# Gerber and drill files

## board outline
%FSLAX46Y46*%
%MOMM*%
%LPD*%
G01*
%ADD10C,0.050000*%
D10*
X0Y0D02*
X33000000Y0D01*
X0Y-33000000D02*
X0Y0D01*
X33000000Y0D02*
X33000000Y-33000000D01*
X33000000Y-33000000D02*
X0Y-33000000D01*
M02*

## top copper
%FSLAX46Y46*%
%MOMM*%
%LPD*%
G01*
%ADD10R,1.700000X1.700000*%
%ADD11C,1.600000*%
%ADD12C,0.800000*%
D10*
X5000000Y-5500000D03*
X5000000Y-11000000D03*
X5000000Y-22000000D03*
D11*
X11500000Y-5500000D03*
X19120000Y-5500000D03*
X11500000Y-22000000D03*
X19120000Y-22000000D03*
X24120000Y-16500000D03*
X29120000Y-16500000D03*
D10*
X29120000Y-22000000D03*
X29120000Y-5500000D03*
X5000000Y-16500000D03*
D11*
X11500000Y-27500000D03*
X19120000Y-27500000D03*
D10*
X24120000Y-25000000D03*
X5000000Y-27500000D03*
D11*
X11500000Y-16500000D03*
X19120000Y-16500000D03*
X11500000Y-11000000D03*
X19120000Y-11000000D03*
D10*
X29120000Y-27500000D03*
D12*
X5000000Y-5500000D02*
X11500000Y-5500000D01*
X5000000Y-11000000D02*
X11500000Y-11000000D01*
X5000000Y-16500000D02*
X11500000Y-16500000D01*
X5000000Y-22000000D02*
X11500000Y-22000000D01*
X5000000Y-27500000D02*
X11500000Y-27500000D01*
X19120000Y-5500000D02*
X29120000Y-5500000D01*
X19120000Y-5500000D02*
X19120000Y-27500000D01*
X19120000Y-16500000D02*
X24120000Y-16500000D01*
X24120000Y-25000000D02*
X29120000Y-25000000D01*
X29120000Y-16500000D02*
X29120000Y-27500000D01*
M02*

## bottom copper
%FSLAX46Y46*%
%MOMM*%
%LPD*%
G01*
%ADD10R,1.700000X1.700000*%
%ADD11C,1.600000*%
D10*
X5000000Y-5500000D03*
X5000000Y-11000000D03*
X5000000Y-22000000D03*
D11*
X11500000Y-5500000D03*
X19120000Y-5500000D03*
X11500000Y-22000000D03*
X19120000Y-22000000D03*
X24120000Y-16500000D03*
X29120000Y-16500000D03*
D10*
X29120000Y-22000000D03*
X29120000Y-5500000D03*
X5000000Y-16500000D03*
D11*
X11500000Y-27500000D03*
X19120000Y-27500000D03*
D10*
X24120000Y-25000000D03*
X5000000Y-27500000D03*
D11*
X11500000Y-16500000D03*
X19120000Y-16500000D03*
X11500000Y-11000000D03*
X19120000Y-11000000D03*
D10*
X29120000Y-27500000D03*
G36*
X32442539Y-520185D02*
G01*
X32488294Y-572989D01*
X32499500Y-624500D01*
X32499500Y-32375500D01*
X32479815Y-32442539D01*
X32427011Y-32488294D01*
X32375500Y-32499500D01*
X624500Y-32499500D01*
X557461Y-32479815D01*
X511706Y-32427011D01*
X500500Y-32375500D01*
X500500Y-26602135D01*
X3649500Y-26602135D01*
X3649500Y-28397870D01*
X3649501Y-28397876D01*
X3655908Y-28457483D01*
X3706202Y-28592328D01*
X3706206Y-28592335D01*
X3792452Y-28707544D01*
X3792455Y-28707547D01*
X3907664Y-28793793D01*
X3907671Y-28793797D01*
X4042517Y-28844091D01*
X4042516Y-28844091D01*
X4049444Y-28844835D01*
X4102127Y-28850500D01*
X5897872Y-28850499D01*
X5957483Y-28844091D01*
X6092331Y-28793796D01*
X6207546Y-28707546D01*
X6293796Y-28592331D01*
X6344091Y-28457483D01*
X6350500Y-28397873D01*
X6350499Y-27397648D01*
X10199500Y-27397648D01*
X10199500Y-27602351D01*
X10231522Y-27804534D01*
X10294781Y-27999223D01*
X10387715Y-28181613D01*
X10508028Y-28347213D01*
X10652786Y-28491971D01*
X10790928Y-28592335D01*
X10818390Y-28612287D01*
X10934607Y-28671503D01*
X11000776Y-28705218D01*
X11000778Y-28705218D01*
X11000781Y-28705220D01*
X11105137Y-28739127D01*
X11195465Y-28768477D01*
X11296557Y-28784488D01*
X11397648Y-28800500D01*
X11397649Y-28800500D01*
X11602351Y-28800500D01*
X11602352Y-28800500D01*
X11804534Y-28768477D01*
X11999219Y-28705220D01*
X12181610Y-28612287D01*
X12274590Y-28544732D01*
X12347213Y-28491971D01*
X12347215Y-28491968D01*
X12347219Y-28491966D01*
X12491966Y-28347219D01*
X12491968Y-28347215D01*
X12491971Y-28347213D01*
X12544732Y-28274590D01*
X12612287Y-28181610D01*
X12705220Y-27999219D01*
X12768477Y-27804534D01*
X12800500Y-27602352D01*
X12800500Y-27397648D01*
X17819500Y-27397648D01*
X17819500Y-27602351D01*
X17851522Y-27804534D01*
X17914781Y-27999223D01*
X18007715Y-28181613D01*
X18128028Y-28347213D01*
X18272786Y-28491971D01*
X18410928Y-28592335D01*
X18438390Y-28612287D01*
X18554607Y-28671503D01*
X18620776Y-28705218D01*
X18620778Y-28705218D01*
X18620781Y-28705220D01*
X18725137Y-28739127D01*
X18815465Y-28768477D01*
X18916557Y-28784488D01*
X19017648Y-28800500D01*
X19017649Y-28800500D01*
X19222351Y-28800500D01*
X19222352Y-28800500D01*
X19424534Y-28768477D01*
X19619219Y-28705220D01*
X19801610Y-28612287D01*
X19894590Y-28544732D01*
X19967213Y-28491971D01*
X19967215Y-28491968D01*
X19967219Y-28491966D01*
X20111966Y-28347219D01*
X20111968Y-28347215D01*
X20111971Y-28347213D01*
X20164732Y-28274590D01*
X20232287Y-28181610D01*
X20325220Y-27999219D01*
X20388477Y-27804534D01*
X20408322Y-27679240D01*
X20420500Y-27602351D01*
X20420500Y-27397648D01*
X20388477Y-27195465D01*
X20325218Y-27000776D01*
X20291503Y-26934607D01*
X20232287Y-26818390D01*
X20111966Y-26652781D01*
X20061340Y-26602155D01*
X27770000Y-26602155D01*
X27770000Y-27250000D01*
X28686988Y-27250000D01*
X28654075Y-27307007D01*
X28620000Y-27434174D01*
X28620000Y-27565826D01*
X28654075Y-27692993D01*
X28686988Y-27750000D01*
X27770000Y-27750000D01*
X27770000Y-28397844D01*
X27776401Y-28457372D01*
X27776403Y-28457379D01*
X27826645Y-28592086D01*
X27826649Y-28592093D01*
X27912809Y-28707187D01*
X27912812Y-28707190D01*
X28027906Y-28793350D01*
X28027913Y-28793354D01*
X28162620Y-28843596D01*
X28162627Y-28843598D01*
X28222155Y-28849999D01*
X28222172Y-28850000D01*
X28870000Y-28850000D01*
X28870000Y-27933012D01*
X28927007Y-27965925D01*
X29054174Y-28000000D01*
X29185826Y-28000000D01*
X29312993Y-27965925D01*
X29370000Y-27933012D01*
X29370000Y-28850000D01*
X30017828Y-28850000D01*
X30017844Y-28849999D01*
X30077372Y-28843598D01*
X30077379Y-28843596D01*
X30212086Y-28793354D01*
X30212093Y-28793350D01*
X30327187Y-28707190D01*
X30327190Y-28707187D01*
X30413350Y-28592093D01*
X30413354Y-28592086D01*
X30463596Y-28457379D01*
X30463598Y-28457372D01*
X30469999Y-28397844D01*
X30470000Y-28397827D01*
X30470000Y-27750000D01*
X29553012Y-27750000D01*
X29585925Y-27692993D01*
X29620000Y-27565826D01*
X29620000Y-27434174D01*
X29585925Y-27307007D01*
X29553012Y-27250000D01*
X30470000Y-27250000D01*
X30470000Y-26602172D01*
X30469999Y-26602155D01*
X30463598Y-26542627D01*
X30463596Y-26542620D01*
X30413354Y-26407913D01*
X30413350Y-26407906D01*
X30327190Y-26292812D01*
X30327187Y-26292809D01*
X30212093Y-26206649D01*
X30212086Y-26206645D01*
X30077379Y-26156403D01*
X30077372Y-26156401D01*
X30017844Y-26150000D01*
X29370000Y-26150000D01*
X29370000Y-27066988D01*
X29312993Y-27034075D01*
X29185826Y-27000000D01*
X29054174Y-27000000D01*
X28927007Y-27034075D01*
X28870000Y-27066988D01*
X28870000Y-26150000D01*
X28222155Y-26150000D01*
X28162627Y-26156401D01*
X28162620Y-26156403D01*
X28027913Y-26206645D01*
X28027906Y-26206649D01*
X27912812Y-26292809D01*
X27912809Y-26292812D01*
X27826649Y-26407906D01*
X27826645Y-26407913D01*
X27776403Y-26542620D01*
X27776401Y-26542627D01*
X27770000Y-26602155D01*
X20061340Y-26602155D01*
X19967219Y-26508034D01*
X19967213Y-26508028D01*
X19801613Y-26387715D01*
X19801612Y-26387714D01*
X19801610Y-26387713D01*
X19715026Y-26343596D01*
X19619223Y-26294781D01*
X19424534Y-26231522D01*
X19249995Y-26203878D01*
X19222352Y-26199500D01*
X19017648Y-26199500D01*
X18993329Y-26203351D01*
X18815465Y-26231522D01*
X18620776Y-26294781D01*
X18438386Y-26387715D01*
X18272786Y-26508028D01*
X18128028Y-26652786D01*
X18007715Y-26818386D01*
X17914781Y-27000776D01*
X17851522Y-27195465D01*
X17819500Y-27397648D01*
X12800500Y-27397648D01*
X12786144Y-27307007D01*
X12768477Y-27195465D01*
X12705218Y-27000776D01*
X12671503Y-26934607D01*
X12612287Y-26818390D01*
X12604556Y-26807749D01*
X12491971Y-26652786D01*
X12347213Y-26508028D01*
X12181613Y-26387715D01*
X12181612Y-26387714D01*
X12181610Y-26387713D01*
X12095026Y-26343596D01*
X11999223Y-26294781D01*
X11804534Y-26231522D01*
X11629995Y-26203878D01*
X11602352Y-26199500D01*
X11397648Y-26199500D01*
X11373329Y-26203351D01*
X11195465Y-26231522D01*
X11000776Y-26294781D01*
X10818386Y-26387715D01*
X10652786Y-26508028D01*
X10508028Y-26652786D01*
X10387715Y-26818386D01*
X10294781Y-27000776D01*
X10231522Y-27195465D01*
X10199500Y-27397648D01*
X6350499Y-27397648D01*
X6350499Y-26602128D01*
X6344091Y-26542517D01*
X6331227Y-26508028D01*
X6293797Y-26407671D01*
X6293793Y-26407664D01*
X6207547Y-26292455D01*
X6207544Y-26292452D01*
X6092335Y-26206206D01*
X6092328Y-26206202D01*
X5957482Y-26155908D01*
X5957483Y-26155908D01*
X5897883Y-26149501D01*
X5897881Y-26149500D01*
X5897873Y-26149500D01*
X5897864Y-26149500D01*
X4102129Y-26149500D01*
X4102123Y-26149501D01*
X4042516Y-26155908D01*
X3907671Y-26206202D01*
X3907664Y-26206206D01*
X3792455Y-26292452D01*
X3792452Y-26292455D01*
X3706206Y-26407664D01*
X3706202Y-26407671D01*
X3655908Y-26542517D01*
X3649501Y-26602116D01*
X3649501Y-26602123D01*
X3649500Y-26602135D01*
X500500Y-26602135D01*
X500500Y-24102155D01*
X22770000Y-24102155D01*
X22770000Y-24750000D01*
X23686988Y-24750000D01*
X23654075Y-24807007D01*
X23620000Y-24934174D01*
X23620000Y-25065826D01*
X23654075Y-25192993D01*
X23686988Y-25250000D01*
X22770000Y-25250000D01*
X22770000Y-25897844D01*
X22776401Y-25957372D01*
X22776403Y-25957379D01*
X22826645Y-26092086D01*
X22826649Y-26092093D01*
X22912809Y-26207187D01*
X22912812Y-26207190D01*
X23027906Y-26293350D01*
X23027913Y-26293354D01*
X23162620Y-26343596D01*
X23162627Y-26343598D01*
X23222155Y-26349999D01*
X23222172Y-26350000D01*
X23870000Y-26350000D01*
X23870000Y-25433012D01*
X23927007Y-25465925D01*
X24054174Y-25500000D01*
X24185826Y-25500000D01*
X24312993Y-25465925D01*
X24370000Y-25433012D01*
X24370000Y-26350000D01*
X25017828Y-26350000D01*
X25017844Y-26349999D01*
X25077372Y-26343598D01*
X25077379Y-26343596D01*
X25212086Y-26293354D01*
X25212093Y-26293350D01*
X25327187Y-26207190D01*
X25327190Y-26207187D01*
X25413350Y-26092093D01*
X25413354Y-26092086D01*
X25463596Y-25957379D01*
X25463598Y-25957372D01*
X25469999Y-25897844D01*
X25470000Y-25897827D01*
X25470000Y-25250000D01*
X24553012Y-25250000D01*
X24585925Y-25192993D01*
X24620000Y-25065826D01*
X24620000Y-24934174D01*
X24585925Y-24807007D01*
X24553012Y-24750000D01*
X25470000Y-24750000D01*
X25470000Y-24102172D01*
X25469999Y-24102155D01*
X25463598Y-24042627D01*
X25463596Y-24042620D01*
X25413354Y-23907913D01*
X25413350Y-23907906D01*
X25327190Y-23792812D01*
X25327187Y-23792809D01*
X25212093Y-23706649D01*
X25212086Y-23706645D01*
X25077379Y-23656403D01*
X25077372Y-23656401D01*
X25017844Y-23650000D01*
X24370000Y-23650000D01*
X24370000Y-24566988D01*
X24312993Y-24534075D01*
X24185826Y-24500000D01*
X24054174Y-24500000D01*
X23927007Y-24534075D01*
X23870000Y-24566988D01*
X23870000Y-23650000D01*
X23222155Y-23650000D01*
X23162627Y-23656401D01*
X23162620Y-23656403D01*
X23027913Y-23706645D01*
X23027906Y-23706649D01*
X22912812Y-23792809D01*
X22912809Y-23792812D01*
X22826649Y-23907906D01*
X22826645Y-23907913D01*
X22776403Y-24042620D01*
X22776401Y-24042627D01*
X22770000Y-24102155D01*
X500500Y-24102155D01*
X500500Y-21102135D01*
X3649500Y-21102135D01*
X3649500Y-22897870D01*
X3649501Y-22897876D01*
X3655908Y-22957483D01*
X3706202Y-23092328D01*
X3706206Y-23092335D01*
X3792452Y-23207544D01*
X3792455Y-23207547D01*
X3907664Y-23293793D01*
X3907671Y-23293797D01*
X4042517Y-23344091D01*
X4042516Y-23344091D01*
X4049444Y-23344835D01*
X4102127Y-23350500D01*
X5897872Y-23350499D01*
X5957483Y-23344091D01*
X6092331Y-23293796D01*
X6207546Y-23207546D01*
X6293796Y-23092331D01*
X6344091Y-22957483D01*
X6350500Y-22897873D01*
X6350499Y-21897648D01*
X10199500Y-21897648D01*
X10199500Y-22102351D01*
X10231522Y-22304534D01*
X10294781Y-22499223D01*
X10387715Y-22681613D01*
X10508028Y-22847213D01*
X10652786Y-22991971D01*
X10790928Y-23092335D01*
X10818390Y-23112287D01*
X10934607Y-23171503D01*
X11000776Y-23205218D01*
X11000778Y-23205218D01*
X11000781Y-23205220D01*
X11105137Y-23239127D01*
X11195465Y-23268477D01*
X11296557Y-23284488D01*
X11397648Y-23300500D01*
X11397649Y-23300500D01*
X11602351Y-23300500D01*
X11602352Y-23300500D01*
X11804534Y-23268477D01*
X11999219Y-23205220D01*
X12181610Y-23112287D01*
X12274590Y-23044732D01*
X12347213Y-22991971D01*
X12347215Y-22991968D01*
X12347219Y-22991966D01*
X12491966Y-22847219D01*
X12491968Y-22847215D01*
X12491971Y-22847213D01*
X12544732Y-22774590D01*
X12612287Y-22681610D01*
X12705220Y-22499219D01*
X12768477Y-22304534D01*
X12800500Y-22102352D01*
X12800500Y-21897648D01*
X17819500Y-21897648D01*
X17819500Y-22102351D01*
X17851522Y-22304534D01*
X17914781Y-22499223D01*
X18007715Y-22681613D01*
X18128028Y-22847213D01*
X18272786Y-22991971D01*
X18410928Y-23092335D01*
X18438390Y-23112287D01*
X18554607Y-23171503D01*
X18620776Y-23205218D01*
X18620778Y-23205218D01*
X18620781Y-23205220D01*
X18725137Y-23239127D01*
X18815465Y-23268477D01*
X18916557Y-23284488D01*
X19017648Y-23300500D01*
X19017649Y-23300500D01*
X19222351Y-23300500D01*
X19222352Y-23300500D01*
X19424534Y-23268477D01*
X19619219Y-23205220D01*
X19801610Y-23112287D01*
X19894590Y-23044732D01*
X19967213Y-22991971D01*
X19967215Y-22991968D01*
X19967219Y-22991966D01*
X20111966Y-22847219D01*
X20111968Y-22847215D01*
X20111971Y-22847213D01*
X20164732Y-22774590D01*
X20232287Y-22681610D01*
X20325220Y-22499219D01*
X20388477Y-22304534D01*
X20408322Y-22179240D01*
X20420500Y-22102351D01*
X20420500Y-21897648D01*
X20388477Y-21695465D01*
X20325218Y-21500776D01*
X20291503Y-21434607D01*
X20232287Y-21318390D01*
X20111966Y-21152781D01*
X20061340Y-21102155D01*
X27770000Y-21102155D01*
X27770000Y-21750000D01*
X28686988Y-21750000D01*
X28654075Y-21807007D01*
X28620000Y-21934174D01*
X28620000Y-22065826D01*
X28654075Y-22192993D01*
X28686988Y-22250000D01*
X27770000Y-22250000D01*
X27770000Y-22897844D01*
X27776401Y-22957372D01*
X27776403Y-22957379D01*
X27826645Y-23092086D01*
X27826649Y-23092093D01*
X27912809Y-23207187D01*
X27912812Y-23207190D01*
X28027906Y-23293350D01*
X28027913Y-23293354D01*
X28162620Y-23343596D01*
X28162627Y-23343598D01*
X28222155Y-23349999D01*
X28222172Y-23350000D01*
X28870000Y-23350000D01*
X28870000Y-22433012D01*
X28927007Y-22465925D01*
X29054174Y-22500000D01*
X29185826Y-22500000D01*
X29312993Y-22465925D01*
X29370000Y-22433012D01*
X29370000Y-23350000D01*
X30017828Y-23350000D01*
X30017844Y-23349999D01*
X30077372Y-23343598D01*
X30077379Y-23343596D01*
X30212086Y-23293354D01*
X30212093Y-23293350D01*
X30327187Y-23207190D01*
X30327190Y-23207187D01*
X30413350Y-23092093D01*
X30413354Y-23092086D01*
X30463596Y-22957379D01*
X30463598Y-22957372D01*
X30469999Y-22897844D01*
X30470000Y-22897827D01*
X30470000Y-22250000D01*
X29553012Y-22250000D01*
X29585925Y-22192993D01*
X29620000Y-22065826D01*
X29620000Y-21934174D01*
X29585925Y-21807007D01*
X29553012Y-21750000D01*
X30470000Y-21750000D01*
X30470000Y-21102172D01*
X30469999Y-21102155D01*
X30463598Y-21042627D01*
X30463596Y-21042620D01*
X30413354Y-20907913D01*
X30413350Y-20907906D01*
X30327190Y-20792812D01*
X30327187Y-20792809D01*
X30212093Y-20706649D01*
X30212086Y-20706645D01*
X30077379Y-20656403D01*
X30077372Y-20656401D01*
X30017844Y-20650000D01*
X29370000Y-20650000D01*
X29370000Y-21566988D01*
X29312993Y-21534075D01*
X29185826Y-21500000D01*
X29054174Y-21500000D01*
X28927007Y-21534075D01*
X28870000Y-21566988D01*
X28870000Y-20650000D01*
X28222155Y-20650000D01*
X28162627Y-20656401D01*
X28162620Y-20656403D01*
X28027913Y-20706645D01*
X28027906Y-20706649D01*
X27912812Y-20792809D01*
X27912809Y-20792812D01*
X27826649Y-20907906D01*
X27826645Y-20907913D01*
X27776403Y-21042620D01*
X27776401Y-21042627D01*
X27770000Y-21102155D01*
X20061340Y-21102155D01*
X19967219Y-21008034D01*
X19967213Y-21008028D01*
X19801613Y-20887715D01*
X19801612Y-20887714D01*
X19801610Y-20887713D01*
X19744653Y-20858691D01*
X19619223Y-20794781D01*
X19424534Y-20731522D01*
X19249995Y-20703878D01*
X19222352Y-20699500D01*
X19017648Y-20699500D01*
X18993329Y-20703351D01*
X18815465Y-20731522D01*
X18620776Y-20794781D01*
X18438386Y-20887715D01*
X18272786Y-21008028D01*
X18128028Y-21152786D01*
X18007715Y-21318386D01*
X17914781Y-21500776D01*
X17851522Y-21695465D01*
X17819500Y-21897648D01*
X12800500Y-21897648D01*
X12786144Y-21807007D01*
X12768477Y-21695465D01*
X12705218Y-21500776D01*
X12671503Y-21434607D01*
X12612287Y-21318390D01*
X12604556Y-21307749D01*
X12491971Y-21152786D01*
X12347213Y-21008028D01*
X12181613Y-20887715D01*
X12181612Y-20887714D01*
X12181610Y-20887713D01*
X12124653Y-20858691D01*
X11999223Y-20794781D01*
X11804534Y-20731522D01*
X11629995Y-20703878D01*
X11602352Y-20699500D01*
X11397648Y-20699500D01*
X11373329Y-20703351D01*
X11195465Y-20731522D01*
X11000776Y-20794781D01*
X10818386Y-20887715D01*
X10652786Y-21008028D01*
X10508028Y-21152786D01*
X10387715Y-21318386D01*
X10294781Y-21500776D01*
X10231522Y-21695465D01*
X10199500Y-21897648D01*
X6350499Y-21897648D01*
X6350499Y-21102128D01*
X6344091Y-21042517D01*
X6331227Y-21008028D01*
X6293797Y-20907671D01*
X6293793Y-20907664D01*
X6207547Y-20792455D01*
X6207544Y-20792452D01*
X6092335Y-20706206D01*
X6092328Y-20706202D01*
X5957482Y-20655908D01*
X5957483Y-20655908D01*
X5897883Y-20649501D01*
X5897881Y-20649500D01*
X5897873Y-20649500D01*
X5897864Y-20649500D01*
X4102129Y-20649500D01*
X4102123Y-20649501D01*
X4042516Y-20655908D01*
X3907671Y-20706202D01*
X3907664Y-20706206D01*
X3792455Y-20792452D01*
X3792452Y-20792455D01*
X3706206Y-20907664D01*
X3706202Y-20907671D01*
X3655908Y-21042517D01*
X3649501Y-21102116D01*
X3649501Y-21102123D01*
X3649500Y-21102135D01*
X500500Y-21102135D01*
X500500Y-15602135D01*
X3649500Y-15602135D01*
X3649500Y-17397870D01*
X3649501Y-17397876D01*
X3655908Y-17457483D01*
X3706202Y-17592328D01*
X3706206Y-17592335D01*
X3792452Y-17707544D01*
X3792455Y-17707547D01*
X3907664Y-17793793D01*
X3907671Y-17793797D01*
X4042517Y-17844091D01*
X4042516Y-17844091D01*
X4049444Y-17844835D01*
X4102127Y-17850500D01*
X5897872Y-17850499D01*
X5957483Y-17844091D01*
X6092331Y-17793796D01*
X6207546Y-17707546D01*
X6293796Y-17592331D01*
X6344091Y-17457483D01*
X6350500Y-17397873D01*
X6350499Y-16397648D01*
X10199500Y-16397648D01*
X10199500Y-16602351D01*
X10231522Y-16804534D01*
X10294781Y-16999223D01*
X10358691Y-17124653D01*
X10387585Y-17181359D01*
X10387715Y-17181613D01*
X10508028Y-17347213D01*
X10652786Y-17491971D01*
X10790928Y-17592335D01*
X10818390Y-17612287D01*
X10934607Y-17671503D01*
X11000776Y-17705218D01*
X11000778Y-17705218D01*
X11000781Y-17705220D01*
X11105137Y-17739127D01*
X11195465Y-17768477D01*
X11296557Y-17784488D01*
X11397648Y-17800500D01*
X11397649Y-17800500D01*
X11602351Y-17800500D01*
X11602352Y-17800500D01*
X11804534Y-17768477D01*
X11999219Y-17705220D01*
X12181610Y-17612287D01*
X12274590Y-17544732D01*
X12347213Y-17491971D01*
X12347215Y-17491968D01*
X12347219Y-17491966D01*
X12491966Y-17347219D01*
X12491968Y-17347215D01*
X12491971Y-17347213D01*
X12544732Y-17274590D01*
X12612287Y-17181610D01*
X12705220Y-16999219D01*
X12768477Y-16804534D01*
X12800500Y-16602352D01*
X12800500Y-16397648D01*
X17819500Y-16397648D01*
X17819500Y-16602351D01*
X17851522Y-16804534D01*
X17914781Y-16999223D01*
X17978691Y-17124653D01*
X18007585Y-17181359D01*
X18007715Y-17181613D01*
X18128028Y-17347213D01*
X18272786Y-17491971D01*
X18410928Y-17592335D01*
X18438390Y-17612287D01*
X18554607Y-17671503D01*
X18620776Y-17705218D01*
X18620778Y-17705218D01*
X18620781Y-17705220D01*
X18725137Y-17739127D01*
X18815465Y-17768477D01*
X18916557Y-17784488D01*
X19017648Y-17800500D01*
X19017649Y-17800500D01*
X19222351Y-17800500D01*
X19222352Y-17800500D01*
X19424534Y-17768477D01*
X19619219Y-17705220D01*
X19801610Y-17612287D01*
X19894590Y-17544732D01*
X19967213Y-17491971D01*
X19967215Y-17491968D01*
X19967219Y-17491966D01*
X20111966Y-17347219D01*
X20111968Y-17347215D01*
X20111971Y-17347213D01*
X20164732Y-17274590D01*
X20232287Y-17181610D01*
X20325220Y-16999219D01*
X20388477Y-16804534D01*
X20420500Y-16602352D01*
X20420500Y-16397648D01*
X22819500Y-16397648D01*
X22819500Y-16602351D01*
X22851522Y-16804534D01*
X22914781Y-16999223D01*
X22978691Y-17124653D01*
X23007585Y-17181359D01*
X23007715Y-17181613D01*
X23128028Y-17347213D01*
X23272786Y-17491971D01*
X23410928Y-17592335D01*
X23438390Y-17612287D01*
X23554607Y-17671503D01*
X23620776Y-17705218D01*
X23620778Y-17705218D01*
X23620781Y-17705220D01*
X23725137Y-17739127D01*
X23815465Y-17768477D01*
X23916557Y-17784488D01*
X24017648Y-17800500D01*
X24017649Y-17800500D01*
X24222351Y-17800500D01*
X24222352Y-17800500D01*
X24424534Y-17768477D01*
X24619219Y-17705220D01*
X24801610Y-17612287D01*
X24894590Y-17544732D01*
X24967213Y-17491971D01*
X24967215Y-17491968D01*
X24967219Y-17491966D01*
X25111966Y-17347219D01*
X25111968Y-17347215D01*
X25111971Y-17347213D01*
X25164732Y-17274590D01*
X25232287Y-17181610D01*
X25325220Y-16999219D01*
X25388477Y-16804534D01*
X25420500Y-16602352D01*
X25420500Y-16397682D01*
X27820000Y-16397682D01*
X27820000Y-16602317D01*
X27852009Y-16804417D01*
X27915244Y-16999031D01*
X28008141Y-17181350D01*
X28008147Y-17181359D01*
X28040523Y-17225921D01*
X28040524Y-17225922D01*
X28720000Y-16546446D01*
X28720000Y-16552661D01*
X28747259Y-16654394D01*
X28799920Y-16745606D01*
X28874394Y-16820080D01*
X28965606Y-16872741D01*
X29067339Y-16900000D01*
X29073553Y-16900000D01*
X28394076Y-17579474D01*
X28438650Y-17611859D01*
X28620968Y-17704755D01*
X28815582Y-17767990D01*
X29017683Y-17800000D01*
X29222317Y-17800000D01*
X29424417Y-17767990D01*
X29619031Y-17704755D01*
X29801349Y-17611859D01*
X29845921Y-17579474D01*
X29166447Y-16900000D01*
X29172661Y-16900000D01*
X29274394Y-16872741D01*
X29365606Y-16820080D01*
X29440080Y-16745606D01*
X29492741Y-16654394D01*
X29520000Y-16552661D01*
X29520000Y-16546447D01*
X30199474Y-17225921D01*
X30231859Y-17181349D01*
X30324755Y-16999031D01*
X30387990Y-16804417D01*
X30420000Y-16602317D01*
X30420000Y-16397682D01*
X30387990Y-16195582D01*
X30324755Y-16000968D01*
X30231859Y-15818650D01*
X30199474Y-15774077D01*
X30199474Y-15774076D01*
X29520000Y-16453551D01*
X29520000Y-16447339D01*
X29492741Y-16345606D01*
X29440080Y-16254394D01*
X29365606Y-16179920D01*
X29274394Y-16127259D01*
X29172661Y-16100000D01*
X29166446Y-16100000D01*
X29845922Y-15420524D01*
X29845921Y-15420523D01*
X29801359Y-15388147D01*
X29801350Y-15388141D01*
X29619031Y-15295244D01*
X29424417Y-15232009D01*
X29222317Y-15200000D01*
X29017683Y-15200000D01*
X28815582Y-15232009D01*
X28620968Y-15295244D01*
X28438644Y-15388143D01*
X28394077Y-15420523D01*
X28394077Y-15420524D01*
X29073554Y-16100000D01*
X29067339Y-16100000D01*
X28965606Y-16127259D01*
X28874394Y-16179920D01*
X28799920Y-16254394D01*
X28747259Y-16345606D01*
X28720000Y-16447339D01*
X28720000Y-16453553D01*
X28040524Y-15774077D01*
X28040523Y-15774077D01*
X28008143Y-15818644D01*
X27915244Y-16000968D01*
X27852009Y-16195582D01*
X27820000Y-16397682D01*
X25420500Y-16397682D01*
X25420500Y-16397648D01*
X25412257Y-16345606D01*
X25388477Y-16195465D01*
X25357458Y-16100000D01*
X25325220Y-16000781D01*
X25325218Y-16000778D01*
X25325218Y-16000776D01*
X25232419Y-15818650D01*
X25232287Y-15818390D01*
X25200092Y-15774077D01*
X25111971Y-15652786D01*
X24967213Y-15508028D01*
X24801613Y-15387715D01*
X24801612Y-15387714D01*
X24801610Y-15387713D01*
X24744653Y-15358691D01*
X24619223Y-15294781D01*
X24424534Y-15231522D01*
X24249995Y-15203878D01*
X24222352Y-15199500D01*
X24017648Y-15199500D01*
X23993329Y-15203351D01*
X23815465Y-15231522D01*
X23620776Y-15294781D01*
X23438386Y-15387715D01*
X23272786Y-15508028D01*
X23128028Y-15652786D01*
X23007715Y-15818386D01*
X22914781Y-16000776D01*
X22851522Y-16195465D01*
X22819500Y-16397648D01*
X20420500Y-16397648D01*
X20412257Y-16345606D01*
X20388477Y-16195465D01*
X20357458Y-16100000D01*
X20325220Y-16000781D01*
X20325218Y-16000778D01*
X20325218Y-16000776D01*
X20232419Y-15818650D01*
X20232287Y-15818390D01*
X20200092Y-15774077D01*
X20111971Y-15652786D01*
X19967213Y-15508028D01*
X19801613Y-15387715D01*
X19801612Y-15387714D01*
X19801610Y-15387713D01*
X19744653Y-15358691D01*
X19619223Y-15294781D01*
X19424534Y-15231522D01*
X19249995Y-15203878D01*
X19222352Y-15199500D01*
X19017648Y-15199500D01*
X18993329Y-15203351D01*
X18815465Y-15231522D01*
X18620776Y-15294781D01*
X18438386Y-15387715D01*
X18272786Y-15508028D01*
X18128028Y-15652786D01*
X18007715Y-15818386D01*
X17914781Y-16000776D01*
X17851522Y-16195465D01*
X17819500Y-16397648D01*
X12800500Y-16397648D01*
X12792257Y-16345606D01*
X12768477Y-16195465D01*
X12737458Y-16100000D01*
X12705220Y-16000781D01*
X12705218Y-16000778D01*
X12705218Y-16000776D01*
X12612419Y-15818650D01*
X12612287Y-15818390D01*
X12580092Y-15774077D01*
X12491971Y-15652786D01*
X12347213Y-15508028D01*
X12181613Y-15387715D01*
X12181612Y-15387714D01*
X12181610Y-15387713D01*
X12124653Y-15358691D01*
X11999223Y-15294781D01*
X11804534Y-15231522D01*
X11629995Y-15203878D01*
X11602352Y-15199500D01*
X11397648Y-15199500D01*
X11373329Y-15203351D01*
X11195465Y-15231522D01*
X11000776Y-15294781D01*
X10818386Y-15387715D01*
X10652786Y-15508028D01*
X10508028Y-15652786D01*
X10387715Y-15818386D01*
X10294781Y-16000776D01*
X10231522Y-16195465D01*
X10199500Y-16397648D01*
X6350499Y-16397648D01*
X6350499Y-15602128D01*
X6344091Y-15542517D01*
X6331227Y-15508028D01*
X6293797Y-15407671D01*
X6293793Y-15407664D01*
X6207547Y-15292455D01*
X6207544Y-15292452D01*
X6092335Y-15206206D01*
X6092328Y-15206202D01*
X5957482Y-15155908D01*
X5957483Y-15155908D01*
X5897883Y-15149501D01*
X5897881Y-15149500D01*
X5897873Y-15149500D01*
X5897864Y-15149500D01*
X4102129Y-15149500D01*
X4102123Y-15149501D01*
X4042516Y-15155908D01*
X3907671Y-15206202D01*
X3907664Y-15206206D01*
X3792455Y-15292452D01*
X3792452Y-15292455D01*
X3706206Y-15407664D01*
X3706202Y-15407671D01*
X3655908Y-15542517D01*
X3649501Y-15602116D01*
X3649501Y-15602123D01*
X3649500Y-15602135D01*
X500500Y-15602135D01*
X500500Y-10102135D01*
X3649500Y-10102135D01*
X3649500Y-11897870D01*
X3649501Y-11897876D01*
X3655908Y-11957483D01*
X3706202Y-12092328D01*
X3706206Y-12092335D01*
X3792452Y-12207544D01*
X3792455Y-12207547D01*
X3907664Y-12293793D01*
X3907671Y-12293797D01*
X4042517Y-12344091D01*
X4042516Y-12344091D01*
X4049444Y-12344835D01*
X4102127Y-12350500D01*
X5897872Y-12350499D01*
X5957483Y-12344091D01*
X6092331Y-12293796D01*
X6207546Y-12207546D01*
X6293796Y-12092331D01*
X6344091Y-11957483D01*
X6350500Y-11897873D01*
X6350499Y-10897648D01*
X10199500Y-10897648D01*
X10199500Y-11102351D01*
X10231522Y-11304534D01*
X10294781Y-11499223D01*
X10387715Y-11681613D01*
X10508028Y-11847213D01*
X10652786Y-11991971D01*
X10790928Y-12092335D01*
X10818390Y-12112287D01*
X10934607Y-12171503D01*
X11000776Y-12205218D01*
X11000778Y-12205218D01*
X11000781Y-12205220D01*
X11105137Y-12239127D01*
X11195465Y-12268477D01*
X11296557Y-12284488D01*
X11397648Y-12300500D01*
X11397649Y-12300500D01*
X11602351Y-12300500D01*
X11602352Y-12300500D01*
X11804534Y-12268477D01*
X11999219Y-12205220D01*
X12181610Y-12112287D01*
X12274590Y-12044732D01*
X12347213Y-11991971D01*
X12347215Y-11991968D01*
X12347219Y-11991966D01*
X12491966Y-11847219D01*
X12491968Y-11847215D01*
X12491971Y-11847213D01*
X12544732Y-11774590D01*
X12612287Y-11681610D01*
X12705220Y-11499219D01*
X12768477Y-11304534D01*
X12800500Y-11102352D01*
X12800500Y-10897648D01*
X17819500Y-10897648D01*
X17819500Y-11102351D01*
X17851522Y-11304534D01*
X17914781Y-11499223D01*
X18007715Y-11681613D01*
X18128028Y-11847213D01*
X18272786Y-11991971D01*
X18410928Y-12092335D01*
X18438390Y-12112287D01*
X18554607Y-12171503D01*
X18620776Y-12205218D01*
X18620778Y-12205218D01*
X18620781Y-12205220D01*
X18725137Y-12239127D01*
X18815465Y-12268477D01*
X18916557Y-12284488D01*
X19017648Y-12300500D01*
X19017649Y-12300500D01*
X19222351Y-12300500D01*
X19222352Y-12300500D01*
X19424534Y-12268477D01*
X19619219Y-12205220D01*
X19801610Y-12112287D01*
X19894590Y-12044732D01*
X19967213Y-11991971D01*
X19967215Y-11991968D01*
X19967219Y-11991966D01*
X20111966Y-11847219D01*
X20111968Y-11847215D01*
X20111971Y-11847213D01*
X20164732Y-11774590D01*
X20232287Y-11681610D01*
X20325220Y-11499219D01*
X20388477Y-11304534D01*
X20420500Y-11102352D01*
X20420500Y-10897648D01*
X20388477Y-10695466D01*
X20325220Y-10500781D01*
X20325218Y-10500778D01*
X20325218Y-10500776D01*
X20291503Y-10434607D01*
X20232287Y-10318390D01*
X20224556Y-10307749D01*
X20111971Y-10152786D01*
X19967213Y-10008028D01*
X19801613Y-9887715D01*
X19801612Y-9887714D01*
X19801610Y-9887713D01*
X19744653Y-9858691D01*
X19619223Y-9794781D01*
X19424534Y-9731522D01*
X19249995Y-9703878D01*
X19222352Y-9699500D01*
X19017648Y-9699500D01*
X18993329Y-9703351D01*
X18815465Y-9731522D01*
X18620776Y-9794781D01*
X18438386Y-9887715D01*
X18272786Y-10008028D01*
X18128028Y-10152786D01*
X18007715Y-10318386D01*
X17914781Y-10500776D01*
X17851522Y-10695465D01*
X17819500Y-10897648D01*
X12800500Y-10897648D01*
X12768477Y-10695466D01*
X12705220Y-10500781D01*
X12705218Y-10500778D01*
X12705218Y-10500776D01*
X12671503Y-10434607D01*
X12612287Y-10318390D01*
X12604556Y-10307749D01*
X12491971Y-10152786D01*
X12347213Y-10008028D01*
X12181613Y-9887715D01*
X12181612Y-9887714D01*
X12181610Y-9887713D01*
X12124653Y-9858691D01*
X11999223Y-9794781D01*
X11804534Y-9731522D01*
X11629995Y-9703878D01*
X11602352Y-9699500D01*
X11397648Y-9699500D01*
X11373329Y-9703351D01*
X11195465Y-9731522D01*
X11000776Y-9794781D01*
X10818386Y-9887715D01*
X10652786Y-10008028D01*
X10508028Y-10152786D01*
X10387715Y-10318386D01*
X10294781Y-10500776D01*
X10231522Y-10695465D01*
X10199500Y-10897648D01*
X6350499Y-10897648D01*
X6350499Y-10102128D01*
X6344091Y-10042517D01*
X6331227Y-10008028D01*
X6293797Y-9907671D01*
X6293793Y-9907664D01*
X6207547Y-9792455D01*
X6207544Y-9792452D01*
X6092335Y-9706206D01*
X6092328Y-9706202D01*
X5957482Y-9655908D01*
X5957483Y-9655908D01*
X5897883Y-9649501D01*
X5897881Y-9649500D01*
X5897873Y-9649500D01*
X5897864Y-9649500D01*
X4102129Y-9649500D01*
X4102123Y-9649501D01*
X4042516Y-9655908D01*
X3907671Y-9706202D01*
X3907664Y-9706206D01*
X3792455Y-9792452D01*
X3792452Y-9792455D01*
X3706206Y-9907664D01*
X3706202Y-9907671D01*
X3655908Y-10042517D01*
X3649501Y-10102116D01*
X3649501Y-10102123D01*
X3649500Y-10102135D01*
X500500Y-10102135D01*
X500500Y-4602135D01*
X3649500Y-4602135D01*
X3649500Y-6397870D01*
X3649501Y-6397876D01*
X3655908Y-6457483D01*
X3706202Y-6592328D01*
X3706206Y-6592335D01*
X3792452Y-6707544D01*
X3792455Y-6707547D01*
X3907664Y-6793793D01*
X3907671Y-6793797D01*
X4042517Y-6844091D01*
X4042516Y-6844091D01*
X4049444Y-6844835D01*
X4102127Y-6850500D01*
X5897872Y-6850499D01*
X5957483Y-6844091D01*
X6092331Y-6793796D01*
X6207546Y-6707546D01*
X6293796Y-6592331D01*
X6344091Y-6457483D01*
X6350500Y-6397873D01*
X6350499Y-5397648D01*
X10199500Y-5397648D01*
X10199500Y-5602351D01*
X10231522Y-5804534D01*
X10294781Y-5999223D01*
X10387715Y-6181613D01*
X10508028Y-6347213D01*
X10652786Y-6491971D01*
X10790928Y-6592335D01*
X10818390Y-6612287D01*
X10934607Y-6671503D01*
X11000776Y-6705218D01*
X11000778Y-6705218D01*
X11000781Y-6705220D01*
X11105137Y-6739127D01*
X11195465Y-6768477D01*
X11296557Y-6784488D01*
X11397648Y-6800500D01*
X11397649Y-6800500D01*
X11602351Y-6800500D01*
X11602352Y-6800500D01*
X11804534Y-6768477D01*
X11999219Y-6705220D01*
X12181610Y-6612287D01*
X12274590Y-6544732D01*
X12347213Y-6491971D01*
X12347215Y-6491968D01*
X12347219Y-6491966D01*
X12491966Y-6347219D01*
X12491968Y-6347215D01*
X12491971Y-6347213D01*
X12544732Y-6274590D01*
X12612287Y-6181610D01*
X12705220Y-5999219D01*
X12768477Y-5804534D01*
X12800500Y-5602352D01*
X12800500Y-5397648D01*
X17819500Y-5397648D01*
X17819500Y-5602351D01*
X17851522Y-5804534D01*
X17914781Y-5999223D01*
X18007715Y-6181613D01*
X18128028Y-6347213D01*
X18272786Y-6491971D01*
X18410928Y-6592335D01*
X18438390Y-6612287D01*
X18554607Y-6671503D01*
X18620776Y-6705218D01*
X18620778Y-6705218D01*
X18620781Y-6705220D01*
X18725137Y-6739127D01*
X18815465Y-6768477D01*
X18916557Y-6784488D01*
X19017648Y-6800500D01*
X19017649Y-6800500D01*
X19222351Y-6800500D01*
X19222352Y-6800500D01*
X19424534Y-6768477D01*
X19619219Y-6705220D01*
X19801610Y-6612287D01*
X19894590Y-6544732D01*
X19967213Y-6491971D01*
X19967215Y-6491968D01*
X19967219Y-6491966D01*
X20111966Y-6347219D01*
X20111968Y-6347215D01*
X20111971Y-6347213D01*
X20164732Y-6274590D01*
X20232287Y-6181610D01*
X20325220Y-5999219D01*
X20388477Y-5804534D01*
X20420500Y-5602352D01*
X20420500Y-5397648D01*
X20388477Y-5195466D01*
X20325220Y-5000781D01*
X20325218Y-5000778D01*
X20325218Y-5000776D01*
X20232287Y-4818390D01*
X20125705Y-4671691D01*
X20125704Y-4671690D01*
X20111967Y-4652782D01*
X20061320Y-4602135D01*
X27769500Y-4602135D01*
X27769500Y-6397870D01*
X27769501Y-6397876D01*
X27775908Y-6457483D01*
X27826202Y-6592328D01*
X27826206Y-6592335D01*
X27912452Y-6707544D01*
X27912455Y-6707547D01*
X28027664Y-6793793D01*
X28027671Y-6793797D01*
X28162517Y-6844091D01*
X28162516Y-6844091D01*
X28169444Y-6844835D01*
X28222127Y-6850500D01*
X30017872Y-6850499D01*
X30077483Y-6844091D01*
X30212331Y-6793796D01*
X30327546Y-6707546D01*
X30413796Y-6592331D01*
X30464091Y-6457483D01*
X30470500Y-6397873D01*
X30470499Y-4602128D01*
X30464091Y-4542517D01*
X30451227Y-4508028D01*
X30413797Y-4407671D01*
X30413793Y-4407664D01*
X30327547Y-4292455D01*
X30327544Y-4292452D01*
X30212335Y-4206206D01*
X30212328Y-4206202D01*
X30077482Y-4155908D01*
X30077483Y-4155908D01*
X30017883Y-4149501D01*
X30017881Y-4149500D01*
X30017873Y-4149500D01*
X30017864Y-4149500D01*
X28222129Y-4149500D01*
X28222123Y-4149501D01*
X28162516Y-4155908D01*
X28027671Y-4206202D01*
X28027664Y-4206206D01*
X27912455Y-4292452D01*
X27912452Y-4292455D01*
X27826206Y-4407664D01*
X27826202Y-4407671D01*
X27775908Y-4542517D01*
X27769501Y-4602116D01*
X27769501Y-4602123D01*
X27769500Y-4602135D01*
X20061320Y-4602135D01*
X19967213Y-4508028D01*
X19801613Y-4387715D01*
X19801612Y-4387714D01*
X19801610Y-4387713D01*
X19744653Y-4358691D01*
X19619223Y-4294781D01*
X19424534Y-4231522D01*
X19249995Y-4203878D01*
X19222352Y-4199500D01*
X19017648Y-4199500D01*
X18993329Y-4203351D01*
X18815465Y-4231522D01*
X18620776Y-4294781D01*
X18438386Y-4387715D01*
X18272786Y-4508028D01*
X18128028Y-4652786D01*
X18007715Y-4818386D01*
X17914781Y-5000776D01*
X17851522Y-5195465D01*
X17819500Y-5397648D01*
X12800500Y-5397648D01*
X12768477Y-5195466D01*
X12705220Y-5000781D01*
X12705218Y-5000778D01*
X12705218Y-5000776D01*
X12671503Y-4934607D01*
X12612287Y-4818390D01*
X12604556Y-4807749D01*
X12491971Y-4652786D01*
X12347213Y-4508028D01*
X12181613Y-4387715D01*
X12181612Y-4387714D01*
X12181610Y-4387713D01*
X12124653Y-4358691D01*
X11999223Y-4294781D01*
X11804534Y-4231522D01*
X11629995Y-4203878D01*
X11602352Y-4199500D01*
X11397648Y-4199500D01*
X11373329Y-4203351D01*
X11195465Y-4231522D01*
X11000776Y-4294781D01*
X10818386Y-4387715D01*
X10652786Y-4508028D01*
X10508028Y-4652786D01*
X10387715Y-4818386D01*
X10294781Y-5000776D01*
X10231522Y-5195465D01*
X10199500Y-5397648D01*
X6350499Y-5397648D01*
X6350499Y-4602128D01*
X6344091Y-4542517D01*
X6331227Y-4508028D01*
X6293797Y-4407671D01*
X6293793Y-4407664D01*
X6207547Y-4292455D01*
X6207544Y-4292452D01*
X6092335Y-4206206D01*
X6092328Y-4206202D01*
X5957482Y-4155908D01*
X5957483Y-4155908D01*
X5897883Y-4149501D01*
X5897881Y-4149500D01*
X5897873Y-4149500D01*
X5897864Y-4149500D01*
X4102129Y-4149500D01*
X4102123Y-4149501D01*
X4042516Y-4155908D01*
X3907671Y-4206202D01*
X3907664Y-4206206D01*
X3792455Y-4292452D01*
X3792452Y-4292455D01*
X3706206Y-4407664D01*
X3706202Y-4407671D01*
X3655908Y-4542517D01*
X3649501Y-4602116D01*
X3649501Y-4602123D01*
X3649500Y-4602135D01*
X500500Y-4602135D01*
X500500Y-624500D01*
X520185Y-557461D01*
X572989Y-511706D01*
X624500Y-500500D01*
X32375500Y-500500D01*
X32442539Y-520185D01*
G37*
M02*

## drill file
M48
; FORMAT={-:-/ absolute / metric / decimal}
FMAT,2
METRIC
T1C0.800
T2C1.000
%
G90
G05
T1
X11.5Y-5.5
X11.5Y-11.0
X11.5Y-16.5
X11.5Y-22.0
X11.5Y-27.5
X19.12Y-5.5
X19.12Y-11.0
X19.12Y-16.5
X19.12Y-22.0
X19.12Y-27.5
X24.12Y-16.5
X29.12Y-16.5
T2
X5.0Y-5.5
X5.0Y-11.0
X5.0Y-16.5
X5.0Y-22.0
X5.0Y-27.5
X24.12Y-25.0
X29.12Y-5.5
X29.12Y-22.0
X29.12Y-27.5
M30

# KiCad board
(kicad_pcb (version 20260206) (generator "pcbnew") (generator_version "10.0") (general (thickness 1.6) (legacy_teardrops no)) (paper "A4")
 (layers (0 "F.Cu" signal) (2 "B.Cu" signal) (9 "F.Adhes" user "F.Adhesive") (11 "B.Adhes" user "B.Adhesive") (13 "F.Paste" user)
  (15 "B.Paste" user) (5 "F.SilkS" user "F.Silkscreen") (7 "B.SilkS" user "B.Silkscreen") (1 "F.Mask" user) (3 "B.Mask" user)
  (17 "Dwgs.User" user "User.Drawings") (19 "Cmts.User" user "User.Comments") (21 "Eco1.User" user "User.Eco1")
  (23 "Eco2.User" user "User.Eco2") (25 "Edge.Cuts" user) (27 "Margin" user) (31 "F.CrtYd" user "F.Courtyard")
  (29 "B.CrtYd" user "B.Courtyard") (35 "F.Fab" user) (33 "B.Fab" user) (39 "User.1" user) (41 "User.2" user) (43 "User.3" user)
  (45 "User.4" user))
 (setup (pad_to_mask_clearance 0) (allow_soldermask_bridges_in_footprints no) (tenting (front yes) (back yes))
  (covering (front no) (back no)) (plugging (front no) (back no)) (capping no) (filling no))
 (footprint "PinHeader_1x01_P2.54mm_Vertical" (layer "F.Cu") (at 5 5.5)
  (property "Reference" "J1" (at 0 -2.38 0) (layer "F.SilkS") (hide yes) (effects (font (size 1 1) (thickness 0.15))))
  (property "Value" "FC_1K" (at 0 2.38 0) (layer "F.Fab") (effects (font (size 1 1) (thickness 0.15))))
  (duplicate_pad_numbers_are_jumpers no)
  (pad "1" thru_hole rect (at 0 0) (size 1.7 1.7) (drill 1) (layers "*.Cu" "*.Mask") (remove_unused_layers no) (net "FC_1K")))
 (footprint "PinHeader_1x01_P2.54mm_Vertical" (layer "F.Cu") (at 5 11)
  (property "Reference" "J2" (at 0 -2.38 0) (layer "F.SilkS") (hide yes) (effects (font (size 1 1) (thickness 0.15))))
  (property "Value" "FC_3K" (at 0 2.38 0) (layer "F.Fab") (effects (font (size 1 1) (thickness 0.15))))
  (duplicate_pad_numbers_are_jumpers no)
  (pad "1" thru_hole rect (at 0 0) (size 1.7 1.7) (drill 1) (layers "*.Cu" "*.Mask") (remove_unused_layers no) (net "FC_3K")))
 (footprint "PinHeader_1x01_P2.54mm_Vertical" (layer "F.Cu") (at 5 22)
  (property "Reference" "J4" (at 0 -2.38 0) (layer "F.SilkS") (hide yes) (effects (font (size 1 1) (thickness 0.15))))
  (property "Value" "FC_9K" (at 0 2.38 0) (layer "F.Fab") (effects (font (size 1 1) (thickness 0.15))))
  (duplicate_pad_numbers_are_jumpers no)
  (pad "1" thru_hole rect (at 0 0) (size 1.7 1.7) (drill 1) (layers "*.Cu" "*.Mask") (remove_unused_layers no) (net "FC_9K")))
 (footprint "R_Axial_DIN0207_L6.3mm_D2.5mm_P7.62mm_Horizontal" (layer "F.Cu") (at 11.5 5.5)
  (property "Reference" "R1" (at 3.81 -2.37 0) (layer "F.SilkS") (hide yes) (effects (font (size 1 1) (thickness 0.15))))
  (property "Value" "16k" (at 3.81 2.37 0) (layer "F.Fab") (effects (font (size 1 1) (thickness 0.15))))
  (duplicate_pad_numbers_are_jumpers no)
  (pad "1" thru_hole circle (at 0 0) (size 1.6 1.6) (drill 0.8) (layers "*.Cu" "*.Mask") (remove_unused_layers no) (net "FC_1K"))
  (pad "2" thru_hole circle (at 7.62 0) (size 1.6 1.6) (drill 0.8) (layers "*.Cu" "*.Mask") (remove_unused_layers no) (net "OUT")))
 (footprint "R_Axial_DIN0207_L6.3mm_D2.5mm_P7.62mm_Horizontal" (layer "F.Cu") (at 11.5 22)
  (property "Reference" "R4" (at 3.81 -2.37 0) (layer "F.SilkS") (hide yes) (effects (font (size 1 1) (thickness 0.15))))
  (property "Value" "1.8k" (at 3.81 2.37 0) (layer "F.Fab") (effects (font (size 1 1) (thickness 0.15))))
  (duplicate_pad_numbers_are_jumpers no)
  (pad "1" thru_hole circle (at 0 0) (size 1.6 1.6) (drill 0.8) (layers "*.Cu" "*.Mask") (remove_unused_layers no) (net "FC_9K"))
  (pad "2" thru_hole circle (at 7.62 0) (size 1.6 1.6) (drill 0.8) (layers "*.Cu" "*.Mask") (remove_unused_layers no) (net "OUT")))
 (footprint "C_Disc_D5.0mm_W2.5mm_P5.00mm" (layer "F.Cu") (at 24.12 16.5)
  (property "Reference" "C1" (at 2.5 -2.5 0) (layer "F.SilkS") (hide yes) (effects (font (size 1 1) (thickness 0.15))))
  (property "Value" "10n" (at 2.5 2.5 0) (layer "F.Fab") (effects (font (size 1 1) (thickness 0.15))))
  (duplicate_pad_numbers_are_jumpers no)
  (pad "1" thru_hole circle (at 0 0) (size 1.6 1.6) (drill 0.8) (layers "*.Cu" "*.Mask") (remove_unused_layers no) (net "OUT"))
  (pad "2" thru_hole circle (at 5 0) (size 1.6 1.6) (drill 0.8) (layers "*.Cu" "*.Mask") (remove_unused_layers no) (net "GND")))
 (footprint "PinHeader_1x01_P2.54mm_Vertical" (layer "F.Cu") (at 29.12 22)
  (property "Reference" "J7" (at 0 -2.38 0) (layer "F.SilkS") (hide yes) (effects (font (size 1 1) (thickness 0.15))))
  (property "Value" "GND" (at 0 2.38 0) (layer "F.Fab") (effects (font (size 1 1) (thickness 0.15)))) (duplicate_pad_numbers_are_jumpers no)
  (pad "1" thru_hole rect (at 0 0) (size 1.7 1.7) (drill 1) (layers "*.Cu" "*.Mask") (remove_unused_layers no) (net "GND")))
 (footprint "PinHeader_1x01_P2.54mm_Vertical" (layer "F.Cu") (at 29.12 5.5)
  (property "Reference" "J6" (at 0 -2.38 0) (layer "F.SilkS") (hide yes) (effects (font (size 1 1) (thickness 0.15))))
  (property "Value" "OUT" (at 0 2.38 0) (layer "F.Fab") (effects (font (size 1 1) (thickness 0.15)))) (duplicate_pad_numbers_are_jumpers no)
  (pad "1" thru_hole rect (at 0 0) (size 1.7 1.7) (drill 1) (layers "*.Cu" "*.Mask") (remove_unused_layers no) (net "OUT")))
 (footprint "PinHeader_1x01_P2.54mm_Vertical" (layer "F.Cu") (at 5 16.5)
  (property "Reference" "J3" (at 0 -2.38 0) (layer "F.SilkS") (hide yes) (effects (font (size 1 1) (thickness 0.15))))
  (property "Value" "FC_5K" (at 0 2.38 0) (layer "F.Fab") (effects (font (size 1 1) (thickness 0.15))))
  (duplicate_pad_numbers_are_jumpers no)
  (pad "1" thru_hole rect (at 0 0) (size 1.7 1.7) (drill 1) (layers "*.Cu" "*.Mask") (remove_unused_layers no) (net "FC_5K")))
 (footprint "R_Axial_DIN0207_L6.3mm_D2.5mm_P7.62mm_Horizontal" (layer "F.Cu") (at 11.5 27.5)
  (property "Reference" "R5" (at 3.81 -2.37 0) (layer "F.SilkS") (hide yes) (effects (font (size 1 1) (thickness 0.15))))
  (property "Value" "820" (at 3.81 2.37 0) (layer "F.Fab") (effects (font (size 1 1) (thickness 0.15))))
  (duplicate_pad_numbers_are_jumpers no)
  (pad "1" thru_hole circle (at 0 0) (size 1.6 1.6) (drill 0.8) (layers "*.Cu" "*.Mask") (remove_unused_layers no) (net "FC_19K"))
  (pad "2" thru_hole circle (at 7.62 0) (size 1.6 1.6) (drill 0.8) (layers "*.Cu" "*.Mask") (remove_unused_layers no) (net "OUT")))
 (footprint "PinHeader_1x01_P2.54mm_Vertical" (layer "F.Cu") (at 24.12 25)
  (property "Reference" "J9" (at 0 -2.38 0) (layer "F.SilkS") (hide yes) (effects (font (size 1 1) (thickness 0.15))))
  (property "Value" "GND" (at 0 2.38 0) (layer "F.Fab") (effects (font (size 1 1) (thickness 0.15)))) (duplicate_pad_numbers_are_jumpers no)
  (pad "1" thru_hole rect (at 0 0) (size 1.7 1.7) (drill 1) (layers "*.Cu" "*.Mask") (remove_unused_layers no) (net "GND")))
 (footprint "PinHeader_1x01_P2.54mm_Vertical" (layer "F.Cu") (at 5 27.5)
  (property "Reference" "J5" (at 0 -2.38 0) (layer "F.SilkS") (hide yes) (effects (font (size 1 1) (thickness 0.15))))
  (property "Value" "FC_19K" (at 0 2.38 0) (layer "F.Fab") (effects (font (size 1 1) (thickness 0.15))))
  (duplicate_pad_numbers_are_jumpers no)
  (pad "1" thru_hole rect (at 0 0) (size 1.7 1.7) (drill 1) (layers "*.Cu" "*.Mask") (remove_unused_layers no) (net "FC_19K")))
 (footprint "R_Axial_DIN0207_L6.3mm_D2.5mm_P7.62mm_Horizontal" (layer "F.Cu") (at 11.5 16.5)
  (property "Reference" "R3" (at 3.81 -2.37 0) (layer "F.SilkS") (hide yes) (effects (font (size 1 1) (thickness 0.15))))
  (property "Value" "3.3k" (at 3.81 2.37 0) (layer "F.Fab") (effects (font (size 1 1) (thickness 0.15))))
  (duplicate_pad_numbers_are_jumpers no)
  (pad "1" thru_hole circle (at 0 0) (size 1.6 1.6) (drill 0.8) (layers "*.Cu" "*.Mask") (remove_unused_layers no) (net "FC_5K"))
  (pad "2" thru_hole circle (at 7.62 0) (size 1.6 1.6) (drill 0.8) (layers "*.Cu" "*.Mask") (remove_unused_layers no) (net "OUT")))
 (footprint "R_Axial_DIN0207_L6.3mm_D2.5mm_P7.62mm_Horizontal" (layer "F.Cu") (at 11.5 11)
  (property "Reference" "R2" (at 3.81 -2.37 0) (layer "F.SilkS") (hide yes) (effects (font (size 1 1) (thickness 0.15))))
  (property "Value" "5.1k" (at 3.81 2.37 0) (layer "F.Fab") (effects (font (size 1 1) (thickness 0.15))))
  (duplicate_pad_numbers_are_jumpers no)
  (pad "1" thru_hole circle (at 0 0) (size 1.6 1.6) (drill 0.8) (layers "*.Cu" "*.Mask") (remove_unused_layers no) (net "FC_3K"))
  (pad "2" thru_hole circle (at 7.62 0) (size 1.6 1.6) (drill 0.8) (layers "*.Cu" "*.Mask") (remove_unused_layers no) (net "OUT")))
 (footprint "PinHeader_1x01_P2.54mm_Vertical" (layer "F.Cu") (at 29.12 27.5)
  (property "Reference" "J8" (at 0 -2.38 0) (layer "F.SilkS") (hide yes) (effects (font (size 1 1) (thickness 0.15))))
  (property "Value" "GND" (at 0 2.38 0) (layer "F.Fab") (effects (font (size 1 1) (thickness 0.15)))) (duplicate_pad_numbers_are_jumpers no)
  (pad "1" thru_hole rect (at 0 0) (size 1.7 1.7) (drill 1) (layers "*.Cu" "*.Mask") (remove_unused_layers no) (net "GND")))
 (gr_line (start 0 0) (end 33 0) (stroke (width 0.05) (type default)) (layer "Edge.Cuts"))
 (gr_line (start 0 33) (end 0 0) (stroke (width 0.05) (type default)) (layer "Edge.Cuts"))
 (gr_line (start 33 0) (end 33 33) (stroke (width 0.05) (type default)) (layer "Edge.Cuts"))
 (gr_line (start 33 33) (end 0 33) (stroke (width 0.05) (type default)) (layer "Edge.Cuts"))
 (segment (start 5 5.5) (end 11.5 5.5) (width 0.8) (layer "F.Cu") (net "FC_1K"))
 (segment (start 5 11) (end 11.5 11) (width 0.8) (layer "F.Cu") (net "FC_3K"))
 (segment (start 5 16.5) (end 11.5 16.5) (width 0.8) (layer "F.Cu") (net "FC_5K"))
 (segment (start 5 22) (end 11.5 22) (width 0.8) (layer "F.Cu") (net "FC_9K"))
 (segment (start 5 27.5) (end 11.5 27.5) (width 0.8) (layer "F.Cu") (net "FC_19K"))
 (segment (start 19.12 5.5) (end 29.12 5.5) (width 0.8) (layer "F.Cu") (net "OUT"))
 (segment (start 19.12 5.5) (end 19.12 27.5) (width 0.8) (layer "F.Cu") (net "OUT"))
 (segment (start 19.12 16.5) (end 24.12 16.5) (width 0.8) (layer "F.Cu") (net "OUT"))
 (segment (start 24.12 25) (end 29.12 25) (width 0.8) (layer "F.Cu") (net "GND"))
 (segment (start 29.12 16.5) (end 29.12 27.5) (width 0.8) (layer "F.Cu") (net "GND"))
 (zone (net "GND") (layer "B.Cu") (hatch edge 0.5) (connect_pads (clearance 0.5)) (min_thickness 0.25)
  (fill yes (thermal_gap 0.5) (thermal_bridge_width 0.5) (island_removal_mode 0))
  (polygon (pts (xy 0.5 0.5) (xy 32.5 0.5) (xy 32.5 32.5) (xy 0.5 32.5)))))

